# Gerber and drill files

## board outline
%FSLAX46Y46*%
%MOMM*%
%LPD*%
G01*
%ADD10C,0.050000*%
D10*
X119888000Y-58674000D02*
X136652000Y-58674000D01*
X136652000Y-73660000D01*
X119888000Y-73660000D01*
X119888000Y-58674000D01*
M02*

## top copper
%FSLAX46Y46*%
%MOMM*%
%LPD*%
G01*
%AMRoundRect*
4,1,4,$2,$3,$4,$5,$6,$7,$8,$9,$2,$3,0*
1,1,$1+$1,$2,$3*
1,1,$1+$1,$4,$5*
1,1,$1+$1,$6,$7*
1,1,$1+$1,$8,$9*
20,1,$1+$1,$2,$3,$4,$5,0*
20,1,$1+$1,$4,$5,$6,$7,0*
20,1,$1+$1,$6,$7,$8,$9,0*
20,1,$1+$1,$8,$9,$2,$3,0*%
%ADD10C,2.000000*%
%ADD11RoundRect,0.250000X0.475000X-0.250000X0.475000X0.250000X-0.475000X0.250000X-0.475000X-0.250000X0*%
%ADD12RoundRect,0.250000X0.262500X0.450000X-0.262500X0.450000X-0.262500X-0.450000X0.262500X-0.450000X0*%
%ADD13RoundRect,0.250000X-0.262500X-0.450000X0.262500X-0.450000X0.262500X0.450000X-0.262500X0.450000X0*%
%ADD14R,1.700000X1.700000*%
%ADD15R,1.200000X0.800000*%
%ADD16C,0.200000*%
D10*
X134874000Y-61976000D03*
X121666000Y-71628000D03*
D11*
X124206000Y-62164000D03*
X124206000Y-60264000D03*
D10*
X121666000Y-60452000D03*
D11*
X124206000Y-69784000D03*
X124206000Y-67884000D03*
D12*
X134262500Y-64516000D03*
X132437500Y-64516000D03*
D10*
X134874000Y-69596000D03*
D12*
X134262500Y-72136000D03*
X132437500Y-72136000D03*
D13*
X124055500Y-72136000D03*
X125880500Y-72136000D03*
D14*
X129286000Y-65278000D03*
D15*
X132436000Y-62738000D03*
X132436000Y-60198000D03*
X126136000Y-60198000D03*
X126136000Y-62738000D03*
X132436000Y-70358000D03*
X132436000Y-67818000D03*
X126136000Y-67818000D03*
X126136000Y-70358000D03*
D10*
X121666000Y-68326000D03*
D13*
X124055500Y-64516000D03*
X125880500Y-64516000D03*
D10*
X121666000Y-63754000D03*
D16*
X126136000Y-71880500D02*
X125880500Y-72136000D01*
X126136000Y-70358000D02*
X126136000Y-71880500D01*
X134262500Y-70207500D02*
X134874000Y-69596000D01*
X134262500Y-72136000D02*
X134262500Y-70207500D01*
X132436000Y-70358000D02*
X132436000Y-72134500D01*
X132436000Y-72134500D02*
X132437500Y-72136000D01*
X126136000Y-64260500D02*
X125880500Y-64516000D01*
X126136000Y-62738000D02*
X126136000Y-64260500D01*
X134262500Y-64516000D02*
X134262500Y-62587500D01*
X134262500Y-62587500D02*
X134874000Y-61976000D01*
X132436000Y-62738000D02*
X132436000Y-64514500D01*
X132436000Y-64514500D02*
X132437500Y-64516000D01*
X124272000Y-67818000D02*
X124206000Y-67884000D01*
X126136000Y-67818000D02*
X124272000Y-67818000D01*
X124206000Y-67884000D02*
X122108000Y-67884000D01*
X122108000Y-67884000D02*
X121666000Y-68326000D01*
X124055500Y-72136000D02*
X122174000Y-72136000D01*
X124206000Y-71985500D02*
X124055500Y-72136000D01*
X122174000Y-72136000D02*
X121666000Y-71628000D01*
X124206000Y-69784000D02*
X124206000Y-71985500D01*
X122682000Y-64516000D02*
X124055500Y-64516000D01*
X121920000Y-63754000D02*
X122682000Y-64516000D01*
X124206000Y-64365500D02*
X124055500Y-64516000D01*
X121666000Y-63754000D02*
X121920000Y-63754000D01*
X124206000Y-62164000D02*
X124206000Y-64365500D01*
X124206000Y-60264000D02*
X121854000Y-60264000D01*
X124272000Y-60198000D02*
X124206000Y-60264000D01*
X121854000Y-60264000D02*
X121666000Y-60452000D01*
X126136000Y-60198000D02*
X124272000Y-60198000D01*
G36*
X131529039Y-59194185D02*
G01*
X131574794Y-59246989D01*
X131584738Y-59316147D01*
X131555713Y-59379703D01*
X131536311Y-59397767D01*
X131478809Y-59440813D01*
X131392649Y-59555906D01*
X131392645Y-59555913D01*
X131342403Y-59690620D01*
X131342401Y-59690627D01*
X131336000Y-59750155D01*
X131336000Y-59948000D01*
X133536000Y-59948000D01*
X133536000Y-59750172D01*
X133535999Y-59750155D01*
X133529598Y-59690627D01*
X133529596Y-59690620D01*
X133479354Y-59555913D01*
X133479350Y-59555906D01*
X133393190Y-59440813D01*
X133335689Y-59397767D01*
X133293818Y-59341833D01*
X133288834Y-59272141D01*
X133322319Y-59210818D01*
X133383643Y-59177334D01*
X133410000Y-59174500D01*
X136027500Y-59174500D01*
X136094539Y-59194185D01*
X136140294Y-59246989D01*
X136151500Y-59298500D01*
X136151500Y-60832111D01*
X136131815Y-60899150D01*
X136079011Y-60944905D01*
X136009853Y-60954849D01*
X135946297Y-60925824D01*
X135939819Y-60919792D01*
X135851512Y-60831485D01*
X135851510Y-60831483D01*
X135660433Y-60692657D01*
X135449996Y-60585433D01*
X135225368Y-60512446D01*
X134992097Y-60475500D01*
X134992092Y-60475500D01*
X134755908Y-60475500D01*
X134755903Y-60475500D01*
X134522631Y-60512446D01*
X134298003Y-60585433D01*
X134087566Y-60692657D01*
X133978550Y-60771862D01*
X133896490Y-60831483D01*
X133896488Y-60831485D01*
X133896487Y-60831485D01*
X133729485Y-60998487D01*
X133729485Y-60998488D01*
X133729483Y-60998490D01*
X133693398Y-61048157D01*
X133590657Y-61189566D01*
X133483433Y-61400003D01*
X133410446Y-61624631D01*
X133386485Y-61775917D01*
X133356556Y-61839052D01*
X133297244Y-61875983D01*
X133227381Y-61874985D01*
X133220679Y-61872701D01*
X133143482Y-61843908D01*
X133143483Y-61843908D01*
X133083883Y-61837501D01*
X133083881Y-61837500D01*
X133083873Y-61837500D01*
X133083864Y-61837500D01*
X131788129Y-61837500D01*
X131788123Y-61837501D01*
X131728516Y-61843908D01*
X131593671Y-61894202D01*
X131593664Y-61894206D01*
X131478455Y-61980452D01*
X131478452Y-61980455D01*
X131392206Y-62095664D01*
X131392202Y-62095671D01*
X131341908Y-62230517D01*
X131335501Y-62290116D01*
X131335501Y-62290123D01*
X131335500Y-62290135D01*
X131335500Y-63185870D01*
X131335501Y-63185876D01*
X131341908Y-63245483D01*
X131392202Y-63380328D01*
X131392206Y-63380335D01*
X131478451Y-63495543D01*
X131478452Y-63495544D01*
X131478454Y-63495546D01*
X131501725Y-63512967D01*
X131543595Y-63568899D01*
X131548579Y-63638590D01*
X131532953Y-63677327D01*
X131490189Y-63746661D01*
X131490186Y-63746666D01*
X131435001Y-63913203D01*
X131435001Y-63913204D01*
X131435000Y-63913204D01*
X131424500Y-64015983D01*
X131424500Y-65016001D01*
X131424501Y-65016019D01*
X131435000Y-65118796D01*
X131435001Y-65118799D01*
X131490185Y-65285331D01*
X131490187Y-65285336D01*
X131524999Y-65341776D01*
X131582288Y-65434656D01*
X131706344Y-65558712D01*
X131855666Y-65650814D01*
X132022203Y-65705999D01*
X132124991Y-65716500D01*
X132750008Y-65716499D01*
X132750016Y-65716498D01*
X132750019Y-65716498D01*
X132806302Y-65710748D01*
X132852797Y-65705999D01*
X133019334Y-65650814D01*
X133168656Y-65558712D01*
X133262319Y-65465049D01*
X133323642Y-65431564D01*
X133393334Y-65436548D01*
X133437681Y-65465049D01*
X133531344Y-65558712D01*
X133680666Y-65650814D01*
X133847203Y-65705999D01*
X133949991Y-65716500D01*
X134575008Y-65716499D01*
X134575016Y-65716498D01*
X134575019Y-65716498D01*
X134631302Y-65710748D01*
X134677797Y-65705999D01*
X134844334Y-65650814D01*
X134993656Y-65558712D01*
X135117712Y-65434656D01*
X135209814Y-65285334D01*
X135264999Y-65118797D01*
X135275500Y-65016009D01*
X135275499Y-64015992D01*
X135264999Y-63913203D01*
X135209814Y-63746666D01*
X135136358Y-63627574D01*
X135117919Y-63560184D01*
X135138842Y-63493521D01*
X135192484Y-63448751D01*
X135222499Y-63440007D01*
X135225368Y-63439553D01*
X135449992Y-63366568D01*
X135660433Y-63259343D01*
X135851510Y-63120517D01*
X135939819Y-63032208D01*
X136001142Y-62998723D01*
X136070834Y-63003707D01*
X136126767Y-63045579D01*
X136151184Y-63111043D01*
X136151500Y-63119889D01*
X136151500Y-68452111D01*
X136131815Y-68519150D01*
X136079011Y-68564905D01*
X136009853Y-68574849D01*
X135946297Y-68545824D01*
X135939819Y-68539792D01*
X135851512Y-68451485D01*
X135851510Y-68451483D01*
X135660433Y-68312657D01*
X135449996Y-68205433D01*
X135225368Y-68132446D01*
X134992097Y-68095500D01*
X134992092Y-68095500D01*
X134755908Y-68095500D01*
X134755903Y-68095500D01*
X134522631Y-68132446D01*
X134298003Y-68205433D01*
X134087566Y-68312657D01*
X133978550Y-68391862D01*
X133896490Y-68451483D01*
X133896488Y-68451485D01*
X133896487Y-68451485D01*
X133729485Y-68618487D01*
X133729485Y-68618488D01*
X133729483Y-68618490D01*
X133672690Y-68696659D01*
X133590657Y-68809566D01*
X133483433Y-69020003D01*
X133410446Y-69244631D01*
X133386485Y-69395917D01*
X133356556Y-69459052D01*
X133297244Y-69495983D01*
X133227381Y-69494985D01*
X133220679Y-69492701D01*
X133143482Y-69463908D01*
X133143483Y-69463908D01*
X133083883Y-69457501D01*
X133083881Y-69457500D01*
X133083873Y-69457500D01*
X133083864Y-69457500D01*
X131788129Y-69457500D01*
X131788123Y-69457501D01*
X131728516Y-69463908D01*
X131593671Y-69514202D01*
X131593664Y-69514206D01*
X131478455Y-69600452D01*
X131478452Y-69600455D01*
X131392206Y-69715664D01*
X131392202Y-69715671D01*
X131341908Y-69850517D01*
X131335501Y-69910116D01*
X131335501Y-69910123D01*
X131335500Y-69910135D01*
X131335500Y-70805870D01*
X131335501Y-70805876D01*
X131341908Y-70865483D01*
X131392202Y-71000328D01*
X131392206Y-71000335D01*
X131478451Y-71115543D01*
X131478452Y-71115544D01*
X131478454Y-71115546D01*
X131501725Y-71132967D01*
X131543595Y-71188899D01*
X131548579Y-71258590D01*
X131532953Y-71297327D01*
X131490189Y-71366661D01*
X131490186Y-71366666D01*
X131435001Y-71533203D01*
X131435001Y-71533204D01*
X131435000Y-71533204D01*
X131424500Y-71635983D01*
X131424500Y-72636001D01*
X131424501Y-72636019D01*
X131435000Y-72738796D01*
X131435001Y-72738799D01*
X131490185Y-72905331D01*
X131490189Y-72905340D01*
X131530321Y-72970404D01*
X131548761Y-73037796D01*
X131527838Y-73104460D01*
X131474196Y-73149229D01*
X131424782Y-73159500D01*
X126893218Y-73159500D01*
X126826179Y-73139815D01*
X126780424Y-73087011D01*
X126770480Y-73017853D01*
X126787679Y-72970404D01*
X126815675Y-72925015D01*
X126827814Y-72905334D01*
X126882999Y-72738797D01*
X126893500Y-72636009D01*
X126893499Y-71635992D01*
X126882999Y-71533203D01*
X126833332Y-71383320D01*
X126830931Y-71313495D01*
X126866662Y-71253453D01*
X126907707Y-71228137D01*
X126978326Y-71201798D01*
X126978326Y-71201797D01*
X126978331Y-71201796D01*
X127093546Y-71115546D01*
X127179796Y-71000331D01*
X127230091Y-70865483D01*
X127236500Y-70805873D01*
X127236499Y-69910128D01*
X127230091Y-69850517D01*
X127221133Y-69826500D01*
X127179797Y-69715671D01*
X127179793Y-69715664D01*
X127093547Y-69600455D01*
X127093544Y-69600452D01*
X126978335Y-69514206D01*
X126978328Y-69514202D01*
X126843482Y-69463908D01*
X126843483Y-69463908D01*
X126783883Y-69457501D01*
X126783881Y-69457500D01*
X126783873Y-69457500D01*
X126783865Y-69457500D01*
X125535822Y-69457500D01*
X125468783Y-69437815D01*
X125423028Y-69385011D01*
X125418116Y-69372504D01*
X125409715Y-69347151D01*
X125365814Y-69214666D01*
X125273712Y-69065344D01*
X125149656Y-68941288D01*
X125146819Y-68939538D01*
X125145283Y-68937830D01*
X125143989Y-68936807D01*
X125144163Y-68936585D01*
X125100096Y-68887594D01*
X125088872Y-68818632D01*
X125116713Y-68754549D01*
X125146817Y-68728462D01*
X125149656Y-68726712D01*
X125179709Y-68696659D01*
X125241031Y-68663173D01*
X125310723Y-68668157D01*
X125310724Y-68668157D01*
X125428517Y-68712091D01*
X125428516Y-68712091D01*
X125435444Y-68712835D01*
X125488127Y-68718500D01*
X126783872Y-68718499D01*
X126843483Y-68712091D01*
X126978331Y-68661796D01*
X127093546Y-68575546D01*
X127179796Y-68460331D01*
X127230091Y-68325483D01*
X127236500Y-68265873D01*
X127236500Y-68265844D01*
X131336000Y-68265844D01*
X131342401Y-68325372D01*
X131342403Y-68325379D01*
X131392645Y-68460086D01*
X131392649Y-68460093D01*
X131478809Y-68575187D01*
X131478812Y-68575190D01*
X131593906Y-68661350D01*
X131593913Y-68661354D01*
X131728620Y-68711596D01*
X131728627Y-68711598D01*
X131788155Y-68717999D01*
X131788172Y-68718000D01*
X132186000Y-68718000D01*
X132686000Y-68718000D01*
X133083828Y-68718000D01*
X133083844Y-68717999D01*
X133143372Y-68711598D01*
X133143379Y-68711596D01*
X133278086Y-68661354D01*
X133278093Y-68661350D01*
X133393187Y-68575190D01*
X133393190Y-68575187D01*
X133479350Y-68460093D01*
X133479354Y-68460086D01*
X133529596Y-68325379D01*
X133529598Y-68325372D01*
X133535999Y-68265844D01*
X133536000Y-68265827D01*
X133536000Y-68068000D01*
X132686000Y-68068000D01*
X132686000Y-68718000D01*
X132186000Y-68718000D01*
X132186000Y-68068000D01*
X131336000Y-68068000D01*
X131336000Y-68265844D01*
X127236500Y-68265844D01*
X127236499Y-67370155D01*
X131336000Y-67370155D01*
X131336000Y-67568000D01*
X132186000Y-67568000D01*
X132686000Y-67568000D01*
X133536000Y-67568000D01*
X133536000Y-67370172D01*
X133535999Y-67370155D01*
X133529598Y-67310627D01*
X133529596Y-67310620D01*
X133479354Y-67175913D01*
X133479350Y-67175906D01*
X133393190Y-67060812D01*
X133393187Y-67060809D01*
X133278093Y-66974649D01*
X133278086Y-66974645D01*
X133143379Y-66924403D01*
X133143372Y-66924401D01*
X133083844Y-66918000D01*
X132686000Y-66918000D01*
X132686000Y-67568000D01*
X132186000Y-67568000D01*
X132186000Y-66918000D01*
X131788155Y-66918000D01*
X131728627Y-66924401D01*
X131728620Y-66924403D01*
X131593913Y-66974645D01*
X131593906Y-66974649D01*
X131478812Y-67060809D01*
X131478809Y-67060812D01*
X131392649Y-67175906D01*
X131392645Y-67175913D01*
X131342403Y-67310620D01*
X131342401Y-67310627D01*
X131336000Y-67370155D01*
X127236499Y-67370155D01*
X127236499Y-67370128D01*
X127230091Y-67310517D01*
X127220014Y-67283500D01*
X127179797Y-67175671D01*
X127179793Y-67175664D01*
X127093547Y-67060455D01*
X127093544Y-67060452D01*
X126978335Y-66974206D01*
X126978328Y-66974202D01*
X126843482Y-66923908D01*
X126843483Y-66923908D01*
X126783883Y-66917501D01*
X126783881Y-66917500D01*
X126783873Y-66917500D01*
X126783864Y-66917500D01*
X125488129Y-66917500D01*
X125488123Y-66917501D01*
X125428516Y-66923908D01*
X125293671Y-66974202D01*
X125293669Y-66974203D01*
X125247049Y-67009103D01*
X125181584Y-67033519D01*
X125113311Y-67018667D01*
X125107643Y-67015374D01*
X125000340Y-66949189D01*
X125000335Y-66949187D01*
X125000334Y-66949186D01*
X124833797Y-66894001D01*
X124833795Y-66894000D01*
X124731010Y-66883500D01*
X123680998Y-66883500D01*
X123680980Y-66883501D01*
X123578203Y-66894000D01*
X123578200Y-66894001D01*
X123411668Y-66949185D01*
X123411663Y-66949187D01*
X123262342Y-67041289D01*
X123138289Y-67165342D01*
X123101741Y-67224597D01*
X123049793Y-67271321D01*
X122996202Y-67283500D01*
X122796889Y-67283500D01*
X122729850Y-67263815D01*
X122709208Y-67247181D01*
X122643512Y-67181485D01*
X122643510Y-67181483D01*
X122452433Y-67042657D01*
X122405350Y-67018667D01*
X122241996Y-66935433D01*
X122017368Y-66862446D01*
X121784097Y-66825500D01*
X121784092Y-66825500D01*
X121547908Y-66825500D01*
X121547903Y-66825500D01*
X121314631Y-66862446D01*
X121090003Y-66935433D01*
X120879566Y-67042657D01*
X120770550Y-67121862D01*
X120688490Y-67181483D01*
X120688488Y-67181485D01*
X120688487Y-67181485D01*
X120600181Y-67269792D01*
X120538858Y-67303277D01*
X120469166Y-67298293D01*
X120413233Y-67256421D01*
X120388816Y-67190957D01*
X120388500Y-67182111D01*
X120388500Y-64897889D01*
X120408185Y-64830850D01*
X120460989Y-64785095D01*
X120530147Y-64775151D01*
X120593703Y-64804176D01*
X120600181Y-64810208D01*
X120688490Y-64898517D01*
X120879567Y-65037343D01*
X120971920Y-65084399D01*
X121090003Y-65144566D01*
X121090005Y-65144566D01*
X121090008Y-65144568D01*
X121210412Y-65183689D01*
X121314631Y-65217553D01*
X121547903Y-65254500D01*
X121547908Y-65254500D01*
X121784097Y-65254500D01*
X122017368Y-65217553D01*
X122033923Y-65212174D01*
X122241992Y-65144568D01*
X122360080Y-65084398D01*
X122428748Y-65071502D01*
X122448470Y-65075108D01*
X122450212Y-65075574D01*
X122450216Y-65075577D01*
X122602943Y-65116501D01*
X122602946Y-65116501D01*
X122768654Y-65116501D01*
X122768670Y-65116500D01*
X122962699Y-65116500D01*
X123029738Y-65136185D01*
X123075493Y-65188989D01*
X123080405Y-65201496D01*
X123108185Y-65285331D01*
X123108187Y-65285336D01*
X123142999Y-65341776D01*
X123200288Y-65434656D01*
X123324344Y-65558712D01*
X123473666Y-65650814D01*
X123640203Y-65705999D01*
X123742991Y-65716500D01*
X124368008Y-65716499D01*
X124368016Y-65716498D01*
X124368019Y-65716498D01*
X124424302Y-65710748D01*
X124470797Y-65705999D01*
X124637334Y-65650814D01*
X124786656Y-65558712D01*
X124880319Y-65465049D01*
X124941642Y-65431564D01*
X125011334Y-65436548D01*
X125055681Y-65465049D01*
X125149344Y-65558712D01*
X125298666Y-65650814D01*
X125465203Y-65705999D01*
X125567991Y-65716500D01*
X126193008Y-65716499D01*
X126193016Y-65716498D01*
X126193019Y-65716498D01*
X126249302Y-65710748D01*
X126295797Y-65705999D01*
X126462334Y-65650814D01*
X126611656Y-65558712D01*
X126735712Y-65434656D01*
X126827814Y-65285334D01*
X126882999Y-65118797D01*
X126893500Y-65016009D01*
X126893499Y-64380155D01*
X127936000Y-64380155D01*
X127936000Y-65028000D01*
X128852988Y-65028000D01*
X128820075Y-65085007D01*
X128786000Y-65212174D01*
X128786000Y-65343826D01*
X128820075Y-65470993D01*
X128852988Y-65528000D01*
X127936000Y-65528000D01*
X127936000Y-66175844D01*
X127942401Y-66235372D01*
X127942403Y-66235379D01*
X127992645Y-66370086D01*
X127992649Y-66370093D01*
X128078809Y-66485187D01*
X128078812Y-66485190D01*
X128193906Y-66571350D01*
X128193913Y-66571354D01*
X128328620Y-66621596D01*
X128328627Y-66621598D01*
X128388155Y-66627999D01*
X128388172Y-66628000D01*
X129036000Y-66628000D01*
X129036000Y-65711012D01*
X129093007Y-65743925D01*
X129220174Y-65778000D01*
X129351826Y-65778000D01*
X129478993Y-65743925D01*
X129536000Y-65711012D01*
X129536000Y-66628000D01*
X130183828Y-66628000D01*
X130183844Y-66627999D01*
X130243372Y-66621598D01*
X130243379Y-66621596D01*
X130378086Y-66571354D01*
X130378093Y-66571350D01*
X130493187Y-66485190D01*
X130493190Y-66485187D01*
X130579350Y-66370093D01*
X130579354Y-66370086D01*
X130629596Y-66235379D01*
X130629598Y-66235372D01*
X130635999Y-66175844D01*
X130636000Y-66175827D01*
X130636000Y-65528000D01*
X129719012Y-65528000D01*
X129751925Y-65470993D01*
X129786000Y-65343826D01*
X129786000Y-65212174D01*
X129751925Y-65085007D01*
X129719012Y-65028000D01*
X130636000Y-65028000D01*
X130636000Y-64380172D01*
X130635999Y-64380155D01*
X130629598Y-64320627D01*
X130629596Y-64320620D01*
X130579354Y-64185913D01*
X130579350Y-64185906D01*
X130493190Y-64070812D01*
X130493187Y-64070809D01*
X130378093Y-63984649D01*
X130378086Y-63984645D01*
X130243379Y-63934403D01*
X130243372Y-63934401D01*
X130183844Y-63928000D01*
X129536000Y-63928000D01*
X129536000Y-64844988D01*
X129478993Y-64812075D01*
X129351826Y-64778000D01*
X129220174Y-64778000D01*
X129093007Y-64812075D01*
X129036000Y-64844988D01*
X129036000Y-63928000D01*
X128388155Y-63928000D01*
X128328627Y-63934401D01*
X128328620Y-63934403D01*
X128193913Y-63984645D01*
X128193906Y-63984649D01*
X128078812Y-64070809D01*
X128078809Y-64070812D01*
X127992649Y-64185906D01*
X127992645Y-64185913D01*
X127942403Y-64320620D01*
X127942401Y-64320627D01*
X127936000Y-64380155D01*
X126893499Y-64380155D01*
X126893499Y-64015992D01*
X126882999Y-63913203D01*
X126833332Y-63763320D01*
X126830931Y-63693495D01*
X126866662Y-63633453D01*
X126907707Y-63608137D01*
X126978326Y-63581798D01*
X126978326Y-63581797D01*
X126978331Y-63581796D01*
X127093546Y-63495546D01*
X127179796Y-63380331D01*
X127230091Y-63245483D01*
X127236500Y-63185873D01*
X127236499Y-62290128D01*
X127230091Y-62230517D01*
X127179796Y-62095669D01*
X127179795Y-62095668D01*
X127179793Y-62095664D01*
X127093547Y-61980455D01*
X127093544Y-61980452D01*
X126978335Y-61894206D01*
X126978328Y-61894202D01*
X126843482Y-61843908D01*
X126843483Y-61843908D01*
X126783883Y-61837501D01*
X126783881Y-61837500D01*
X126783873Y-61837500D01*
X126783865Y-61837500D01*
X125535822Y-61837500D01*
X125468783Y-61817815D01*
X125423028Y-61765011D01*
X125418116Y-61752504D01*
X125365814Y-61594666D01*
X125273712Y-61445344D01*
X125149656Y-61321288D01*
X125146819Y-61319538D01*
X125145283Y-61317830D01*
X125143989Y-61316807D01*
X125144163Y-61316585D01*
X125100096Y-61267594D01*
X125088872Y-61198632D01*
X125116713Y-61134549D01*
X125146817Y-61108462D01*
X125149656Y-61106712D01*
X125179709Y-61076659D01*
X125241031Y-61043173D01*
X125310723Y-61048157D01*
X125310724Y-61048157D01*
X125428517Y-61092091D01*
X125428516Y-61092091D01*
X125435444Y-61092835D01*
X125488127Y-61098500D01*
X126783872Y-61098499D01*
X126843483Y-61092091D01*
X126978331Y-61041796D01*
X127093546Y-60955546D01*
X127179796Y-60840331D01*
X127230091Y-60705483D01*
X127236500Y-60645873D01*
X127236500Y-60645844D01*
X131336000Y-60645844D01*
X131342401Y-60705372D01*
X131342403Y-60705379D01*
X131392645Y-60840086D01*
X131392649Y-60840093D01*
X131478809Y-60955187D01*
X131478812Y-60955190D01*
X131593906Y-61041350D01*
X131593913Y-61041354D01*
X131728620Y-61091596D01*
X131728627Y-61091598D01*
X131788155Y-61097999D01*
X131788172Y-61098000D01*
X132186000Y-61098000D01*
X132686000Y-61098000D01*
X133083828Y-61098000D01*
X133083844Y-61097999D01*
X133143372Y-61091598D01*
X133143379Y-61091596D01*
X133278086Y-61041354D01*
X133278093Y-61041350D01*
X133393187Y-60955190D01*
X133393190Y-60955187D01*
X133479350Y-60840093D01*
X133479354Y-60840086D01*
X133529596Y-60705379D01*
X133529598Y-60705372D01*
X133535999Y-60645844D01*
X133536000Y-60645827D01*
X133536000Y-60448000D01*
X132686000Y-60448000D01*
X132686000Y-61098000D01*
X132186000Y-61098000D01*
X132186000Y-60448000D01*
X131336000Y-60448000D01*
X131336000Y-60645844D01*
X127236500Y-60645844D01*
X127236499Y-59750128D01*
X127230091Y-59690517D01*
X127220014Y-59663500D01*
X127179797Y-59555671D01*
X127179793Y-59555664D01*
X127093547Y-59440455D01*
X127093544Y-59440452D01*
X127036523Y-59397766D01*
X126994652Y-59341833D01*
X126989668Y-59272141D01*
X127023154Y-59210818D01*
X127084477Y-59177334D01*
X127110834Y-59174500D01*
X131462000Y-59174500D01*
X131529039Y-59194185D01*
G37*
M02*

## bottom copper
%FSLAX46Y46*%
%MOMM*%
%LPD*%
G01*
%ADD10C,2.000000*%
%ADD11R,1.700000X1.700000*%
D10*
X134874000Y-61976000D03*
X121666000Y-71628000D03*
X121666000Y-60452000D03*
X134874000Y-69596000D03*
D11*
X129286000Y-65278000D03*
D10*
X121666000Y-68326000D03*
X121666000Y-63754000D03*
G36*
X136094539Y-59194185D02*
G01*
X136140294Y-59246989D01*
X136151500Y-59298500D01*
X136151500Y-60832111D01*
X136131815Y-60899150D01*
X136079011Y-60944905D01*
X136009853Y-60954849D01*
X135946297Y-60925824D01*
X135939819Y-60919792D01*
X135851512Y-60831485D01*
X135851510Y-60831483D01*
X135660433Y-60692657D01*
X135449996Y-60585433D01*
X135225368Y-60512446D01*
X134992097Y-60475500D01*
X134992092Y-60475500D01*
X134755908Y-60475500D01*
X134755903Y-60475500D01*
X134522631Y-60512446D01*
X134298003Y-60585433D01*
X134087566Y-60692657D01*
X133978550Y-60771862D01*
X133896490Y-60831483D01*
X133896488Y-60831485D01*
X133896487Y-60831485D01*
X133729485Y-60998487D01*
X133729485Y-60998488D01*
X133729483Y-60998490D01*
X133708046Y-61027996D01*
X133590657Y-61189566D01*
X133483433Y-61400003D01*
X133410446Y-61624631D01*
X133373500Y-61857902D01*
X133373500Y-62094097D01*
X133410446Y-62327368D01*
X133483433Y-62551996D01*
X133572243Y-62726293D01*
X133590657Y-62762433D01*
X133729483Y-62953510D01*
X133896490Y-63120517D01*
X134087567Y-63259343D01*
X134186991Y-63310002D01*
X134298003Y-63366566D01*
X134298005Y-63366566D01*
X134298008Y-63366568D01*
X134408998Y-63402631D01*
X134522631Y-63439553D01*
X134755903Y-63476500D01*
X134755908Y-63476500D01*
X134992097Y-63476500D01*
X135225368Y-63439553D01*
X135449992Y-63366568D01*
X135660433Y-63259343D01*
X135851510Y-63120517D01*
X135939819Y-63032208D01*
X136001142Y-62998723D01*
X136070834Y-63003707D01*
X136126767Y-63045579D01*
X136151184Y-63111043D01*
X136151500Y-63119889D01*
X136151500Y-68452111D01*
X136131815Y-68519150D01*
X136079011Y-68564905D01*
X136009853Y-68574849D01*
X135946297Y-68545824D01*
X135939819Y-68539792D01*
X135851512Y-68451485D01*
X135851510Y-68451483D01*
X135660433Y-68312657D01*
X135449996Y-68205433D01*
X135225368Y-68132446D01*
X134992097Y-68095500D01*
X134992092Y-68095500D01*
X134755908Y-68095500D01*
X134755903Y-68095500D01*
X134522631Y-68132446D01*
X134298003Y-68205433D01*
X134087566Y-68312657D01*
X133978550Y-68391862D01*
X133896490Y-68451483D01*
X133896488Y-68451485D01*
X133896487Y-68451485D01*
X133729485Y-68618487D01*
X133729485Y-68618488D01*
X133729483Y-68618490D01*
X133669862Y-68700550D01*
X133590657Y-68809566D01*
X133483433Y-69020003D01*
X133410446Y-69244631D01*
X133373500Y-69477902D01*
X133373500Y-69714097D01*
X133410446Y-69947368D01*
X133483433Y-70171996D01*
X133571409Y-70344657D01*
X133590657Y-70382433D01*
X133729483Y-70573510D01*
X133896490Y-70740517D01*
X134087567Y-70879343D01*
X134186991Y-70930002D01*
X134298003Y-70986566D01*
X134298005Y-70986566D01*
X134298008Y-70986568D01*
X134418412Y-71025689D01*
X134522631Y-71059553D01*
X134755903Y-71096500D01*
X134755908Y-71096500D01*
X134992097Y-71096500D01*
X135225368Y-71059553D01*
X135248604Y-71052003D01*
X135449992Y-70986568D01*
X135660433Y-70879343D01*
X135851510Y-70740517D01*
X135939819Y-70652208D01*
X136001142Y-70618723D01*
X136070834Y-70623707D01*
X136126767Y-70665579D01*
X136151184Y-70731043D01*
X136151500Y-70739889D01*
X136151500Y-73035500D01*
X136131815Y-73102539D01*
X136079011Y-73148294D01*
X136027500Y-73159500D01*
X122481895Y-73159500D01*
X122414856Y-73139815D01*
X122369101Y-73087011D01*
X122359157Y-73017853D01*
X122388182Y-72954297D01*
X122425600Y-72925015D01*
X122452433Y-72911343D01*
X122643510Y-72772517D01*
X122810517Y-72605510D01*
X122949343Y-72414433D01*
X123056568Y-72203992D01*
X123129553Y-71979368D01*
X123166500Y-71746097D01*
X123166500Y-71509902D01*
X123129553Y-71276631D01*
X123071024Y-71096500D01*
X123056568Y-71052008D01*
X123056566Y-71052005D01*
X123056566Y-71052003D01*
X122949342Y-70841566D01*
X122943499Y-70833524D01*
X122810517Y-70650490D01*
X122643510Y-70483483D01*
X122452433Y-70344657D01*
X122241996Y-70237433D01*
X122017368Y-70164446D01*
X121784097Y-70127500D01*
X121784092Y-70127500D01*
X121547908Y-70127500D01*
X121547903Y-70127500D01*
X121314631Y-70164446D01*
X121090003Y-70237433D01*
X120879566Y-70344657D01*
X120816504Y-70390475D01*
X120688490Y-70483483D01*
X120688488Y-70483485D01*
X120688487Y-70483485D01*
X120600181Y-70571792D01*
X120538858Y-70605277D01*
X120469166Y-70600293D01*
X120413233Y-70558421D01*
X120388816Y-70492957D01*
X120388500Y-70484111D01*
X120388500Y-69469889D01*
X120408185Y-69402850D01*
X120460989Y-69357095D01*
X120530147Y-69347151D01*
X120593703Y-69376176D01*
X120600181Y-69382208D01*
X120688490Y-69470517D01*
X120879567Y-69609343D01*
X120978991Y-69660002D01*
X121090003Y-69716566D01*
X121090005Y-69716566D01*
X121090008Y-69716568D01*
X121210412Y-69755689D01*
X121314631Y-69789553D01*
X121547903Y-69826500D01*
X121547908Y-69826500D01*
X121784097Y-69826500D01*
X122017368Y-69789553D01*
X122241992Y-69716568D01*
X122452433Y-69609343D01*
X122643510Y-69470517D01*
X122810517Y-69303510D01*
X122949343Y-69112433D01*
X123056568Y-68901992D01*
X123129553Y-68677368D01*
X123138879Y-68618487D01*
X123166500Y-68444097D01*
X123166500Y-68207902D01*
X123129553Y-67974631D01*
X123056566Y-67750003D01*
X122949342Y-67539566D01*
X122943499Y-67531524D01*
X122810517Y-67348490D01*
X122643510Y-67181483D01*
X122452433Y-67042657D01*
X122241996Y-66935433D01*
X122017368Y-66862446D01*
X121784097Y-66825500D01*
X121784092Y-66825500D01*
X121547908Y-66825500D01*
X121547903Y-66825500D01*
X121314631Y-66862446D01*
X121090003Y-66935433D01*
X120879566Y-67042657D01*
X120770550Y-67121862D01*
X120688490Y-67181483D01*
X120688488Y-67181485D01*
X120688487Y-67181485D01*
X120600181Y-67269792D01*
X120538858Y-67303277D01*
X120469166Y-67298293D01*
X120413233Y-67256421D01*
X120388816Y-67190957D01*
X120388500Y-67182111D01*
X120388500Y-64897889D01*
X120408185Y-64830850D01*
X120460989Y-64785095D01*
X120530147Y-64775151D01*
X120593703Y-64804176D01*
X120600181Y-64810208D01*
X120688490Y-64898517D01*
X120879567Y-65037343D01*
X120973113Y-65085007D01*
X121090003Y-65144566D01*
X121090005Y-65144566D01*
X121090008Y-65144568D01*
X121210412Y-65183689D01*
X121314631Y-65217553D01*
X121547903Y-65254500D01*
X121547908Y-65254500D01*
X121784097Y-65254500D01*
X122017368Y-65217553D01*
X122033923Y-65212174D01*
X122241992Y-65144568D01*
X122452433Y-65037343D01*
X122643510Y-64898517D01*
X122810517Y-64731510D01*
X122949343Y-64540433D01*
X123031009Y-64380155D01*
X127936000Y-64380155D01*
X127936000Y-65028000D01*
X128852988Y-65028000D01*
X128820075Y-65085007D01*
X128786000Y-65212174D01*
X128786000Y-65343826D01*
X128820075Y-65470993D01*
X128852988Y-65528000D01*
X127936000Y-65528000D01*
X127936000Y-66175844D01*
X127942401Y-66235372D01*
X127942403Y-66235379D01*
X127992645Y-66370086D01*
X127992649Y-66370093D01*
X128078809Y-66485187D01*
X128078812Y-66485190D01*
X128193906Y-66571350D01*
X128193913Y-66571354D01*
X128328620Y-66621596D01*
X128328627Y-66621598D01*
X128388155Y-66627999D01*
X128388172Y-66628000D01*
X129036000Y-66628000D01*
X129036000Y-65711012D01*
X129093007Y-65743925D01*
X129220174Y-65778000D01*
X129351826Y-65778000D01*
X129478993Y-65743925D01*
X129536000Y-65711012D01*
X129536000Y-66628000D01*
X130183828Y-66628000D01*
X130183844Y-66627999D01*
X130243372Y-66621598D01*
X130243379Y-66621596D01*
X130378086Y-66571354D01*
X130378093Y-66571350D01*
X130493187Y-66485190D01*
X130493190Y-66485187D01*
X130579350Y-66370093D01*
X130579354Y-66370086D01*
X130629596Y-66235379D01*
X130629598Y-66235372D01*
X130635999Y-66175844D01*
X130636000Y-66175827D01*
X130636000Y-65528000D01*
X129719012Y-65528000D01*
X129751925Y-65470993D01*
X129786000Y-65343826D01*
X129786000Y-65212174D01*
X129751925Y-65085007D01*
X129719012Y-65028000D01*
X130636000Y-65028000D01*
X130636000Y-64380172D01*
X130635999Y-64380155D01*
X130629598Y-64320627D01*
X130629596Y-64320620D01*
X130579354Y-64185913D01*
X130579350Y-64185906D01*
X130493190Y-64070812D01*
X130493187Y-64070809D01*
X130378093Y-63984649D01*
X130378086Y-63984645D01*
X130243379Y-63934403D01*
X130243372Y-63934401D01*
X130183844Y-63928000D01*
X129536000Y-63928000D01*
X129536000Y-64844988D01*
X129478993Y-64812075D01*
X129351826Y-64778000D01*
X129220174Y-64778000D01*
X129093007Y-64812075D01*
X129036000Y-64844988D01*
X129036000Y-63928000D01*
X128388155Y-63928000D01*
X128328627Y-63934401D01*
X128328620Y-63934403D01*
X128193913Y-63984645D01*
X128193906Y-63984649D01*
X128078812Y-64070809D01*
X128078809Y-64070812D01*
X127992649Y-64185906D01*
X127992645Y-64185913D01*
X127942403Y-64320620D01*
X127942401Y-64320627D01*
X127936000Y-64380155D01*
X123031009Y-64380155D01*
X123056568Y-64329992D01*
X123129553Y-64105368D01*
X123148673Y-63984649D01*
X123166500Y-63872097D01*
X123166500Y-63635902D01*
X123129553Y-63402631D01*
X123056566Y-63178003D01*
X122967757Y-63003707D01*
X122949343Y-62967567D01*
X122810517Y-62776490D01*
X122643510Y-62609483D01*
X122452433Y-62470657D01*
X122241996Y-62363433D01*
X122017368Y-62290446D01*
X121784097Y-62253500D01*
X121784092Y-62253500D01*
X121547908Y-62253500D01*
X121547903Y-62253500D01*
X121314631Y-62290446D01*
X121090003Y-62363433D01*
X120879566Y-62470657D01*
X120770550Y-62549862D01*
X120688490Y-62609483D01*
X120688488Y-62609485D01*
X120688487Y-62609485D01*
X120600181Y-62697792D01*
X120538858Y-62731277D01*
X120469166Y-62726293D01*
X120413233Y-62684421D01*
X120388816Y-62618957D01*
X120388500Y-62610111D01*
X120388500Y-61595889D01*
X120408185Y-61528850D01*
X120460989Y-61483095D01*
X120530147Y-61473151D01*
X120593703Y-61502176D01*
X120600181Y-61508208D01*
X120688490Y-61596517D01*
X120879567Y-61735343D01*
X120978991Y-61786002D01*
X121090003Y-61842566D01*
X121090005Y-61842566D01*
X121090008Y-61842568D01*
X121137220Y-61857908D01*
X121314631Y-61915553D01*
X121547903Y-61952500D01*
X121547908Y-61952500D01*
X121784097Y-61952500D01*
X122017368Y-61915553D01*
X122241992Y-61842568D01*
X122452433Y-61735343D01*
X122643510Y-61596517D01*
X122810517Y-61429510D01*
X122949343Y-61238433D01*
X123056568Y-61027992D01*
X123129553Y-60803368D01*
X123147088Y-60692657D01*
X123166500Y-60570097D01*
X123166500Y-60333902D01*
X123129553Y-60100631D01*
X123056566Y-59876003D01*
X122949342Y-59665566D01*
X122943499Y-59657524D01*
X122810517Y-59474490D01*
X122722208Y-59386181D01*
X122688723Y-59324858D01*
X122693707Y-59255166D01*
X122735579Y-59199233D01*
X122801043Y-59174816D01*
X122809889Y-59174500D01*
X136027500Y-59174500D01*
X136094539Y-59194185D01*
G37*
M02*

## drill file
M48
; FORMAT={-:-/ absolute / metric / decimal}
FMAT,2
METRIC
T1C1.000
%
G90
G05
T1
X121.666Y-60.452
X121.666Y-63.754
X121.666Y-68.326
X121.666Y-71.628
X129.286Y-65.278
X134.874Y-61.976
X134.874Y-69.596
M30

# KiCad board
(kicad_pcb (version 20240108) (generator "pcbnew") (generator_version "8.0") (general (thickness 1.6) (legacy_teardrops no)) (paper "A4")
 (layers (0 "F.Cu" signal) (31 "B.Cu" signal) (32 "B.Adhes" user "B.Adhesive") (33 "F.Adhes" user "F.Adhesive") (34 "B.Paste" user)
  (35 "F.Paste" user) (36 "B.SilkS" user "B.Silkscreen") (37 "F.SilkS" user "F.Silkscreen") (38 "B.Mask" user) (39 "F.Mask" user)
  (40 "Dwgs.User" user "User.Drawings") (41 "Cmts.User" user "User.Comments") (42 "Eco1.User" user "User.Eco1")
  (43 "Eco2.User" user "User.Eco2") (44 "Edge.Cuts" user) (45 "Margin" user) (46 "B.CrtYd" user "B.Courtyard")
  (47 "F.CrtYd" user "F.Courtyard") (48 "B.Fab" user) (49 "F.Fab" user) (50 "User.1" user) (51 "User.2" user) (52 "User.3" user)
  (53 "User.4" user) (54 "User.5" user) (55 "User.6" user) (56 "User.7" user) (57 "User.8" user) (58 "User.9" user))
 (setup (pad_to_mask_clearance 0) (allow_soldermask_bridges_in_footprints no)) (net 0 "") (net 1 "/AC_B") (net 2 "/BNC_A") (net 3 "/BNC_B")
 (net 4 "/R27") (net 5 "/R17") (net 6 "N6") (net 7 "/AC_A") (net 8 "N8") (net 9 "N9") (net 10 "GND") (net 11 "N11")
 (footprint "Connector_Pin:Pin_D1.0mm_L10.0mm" (layer "F.Cu") (at 134.874 61.976 180)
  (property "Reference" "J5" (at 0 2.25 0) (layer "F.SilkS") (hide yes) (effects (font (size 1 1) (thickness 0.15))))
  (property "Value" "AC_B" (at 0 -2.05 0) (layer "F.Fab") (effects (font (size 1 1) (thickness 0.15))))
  (pad "1" thru_hole circle (at 0 0 180) (size 2 2) (drill 1) (layers "*.Cu" "*.Mask") (remove_unused_layers no) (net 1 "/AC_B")))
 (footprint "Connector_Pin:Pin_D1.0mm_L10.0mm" (layer "F.Cu") (at 121.666 71.628 180)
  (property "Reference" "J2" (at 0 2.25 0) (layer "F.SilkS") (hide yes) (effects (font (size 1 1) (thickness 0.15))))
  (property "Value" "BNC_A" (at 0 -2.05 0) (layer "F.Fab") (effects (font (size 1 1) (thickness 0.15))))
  (pad "1" thru_hole circle (at 0 0 180) (size 2 2) (drill 1) (layers "*.Cu" "*.Mask") (remove_unused_layers no) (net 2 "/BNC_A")))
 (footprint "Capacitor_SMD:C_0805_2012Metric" (layer "F.Cu") (at 124.206 61.214 90)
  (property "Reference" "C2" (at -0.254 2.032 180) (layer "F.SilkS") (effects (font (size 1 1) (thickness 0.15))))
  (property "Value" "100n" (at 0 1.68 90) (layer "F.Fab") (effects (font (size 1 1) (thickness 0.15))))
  (pad "1" smd roundrect (at -0.95 0 90) (size 1 1.45) (layers "F.Cu" "F.Paste" "F.Mask") (roundrect_rratio 0.25) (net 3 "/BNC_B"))
  (pad "2" smd roundrect (at 0.95 0 90) (size 1 1.45) (layers "F.Cu" "F.Paste" "F.Mask") (roundrect_rratio 0.25) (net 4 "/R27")))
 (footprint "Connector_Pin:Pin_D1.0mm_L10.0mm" (layer "F.Cu") (at 121.666 60.452 180)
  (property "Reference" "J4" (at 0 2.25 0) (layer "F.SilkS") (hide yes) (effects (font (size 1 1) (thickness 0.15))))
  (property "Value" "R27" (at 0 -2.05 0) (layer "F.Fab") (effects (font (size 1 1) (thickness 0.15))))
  (pad "1" thru_hole circle (at 0 0 180) (size 2 2) (drill 1) (layers "*.Cu" "*.Mask") (remove_unused_layers no) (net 4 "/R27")))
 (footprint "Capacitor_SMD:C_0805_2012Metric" (layer "F.Cu") (at 124.206 68.834 90)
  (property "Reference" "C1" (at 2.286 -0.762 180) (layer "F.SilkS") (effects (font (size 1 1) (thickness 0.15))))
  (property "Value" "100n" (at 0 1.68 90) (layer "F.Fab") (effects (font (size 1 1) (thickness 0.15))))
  (pad "1" smd roundrect (at -0.95 0 90) (size 1 1.45) (layers "F.Cu" "F.Paste" "F.Mask") (roundrect_rratio 0.25) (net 2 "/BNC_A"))
  (pad "2" smd roundrect (at 0.95 0 90) (size 1 1.45) (layers "F.Cu" "F.Paste" "F.Mask") (roundrect_rratio 0.25) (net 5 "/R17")))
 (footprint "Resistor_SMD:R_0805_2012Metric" (layer "F.Cu") (at 133.35 64.516 180)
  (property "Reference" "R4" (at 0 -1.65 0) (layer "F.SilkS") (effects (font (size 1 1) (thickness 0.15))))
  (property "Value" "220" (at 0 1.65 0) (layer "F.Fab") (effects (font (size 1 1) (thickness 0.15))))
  (pad "1" smd roundrect (at -0.9125 0 180) (size 1.025 1.4) (layers "F.Cu" "F.Paste" "F.Mask") (roundrect_rratio 0.243902) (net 1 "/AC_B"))
  (pad "2" smd roundrect (at 0.9125 0 180) (size 1.025 1.4) (layers "F.Cu" "F.Paste" "F.Mask") (roundrect_rratio 0.243902) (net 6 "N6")))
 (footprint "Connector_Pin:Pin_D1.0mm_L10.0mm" (layer "F.Cu") (at 134.874 69.596 180)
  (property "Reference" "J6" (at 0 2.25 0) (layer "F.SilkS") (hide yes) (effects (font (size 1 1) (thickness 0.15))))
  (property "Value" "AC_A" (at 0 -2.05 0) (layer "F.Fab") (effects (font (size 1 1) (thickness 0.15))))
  (pad "1" thru_hole circle (at 0 0 180) (size 2 2) (drill 1) (layers "*.Cu" "*.Mask") (remove_unused_layers no) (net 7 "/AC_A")))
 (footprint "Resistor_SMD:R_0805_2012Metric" (layer "F.Cu") (at 133.35 72.136 180)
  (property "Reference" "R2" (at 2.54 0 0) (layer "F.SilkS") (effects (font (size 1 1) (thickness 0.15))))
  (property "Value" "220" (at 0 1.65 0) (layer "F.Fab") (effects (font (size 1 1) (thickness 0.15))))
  (pad "1" smd roundrect (at -0.9125 0 180) (size 1.025 1.4) (layers "F.Cu" "F.Paste" "F.Mask") (roundrect_rratio 0.243902) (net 7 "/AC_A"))
  (pad "2" smd roundrect (at 0.9125 0 180) (size 1.025 1.4) (layers "F.Cu" "F.Paste" "F.Mask") (roundrect_rratio 0.243902) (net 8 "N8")))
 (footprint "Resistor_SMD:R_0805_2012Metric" (layer "F.Cu") (at 124.968 72.136)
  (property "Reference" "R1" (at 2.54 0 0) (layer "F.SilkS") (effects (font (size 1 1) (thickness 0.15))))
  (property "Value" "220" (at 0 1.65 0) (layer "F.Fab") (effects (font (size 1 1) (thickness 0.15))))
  (pad "1" smd roundrect (at -0.9125 0) (size 1.025 1.4) (layers "F.Cu" "F.Paste" "F.Mask") (roundrect_rratio 0.243902) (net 2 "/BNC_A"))
  (pad "2" smd roundrect (at 0.9125 0) (size 1.025 1.4) (layers "F.Cu" "F.Paste" "F.Mask") (roundrect_rratio 0.243902) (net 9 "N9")))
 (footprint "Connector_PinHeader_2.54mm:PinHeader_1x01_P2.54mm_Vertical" (layer "F.Cu") (at 129.286 65.278)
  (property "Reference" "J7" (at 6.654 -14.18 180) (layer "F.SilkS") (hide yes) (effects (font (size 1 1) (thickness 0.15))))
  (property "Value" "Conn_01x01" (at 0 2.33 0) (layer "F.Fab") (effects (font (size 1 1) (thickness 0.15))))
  (pad "1" thru_hole rect (at 0 0) (size 1.7 1.7) (drill 1) (layers "*.Cu" "*.Mask") (remove_unused_layers no) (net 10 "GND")))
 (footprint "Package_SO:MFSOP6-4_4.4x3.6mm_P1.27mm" (layer "F.Cu") (at 129.286 61.468 180)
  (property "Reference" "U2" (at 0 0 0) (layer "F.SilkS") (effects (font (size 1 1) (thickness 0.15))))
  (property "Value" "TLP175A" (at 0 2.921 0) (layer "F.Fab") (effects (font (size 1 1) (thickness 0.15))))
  (pad "1" smd rect (at -3.15 -1.27 180) (size 1.2 0.8) (layers "F.Cu" "F.Paste" "F.Mask") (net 6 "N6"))
  (pad "3" smd rect (at -3.15 1.27 180) (size 1.2 0.8) (layers "F.Cu" "F.Paste" "F.Mask") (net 10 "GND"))
  (pad "4" smd rect (at 3.15 1.27 180) (size 1.2 0.8) (layers "F.Cu" "F.Paste" "F.Mask") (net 4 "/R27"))
  (pad "6" smd rect (at 3.15 -1.27 180) (size 1.2 0.8) (layers "F.Cu" "F.Paste" "F.Mask") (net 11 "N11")))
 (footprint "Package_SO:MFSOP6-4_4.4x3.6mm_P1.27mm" (layer "F.Cu") (at 129.286 69.088 180)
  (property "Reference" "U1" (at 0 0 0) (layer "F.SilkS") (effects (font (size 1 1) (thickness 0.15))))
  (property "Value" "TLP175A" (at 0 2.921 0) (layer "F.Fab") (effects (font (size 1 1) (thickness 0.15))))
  (pad "1" smd rect (at -3.15 -1.27 180) (size 1.2 0.8) (layers "F.Cu" "F.Paste" "F.Mask") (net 8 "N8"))
  (pad "3" smd rect (at -3.15 1.27 180) (size 1.2 0.8) (layers "F.Cu" "F.Paste" "F.Mask") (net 10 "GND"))
  (pad "4" smd rect (at 3.15 1.27 180) (size 1.2 0.8) (layers "F.Cu" "F.Paste" "F.Mask") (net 5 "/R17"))
  (pad "6" smd rect (at 3.15 -1.27 180) (size 1.2 0.8) (layers "F.Cu" "F.Paste" "F.Mask") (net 9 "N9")))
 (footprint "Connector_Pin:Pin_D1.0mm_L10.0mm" (layer "F.Cu") (at 121.666 68.326 180)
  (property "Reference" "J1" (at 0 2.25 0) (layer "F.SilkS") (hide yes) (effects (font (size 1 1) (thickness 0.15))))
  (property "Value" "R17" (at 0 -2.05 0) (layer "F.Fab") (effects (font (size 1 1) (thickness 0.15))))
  (pad "1" thru_hole circle (at 0 0 180) (size 2 2) (drill 1) (layers "*.Cu" "*.Mask") (remove_unused_layers no) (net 5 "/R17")))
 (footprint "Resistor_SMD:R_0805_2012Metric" (layer "F.Cu") (at 124.968 64.516)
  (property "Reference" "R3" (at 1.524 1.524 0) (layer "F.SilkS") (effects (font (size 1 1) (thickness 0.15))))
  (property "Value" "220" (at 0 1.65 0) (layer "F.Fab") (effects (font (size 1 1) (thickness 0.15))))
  (pad "1" smd roundrect (at -0.9125 0) (size 1.025 1.4) (layers "F.Cu" "F.Paste" "F.Mask") (roundrect_rratio 0.243902) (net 3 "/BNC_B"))
  (pad "2" smd roundrect (at 0.9125 0) (size 1.025 1.4) (layers "F.Cu" "F.Paste" "F.Mask") (roundrect_rratio 0.243902) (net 11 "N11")))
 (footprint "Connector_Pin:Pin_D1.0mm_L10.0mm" (layer "F.Cu") (at 121.666 63.754 180)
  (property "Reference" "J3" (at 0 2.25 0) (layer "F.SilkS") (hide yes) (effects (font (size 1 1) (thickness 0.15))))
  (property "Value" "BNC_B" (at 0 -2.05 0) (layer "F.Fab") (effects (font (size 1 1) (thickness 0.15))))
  (pad "1" thru_hole circle (at 0 0 180) (size 2 2) (drill 1) (layers "*.Cu" "*.Mask") (remove_unused_layers no) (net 3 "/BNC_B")))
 (gr_rect (start 119.888 58.674) (end 136.652 73.66) (stroke (width 0.05) (type default)) (fill none) (layer "Edge.Cuts"))
 (segment (start 126.136 71.8805) (end 125.8805 72.136) (width 0.2) (layer "F.Cu") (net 9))
 (segment (start 126.136 70.358) (end 126.136 71.8805) (width 0.2) (layer "F.Cu") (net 9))
 (segment (start 134.2625 70.2075) (end 134.874 69.596) (width 0.2) (layer "F.Cu") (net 7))
 (segment (start 134.2625 72.136) (end 134.2625 70.2075) (width 0.2) (layer "F.Cu") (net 7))
 (segment (start 132.436 70.358) (end 132.436 72.1345) (width 0.2) (layer "F.Cu") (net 8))
 (segment (start 132.436 72.1345) (end 132.4375 72.136) (width 0.2) (layer "F.Cu") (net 8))
 (segment (start 126.136 64.2605) (end 125.8805 64.516) (width 0.2) (layer "F.Cu") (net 11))
 (segment (start 126.136 62.738) (end 126.136 64.2605) (width 0.2) (layer "F.Cu") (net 11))
 (segment (start 134.2625 64.516) (end 134.2625 62.5875) (width 0.2) (layer "F.Cu") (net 1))
 (segment (start 134.2625 62.5875) (end 134.874 61.976) (width 0.2) (layer "F.Cu") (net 1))
 (segment (start 132.436 62.738) (end 132.436 64.5145) (width 0.2) (layer "F.Cu") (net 6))
 (segment (start 132.436 64.5145) (end 132.4375 64.516) (width 0.2) (layer "F.Cu") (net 6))
 (segment (start 124.272 67.818) (end 124.206 67.884) (width 0.2) (layer "F.Cu") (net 5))
 (segment (start 126.136 67.818) (end 124.272 67.818) (width 0.2) (layer "F.Cu") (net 5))
 (segment (start 124.206 67.884) (end 122.108 67.884) (width 0.2) (layer "F.Cu") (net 5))
 (segment (start 122.108 67.884) (end 121.666 68.326) (width 0.2) (layer "F.Cu") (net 5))
 (segment (start 124.0555 72.136) (end 122.174 72.136) (width 0.2) (layer "F.Cu") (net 2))
 (segment (start 124.206 71.9855) (end 124.0555 72.136) (width 0.2) (layer "F.Cu") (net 2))
 (segment (start 122.174 72.136) (end 121.666 71.628) (width 0.2) (layer "F.Cu") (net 2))
 (segment (start 124.206 69.784) (end 124.206 71.9855) (width 0.2) (layer "F.Cu") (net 2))
 (segment (start 122.682 64.516) (end 124.0555 64.516) (width 0.2) (layer "F.Cu") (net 3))
 (segment (start 121.92 63.754) (end 122.682 64.516) (width 0.2) (layer "F.Cu") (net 3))
 (segment (start 124.206 64.3655) (end 124.0555 64.516) (width 0.2) (layer "F.Cu") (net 3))
 (segment (start 121.666 63.754) (end 121.92 63.754) (width 0.2) (layer "F.Cu") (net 3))
 (segment (start 124.206 62.164) (end 124.206 64.3655) (width 0.2) (layer "F.Cu") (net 3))
 (segment (start 124.206 60.264) (end 121.854 60.264) (width 0.2) (layer "F.Cu") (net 4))
 (segment (start 124.272 60.198) (end 124.206 60.264) (width 0.2) (layer "F.Cu") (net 4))
 (segment (start 121.854 60.264) (end 121.666 60.452) (width 0.2) (layer "F.Cu") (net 4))
 (segment (start 126.136 60.198) (end 124.272 60.198) (width 0.2) (layer "F.Cu") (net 4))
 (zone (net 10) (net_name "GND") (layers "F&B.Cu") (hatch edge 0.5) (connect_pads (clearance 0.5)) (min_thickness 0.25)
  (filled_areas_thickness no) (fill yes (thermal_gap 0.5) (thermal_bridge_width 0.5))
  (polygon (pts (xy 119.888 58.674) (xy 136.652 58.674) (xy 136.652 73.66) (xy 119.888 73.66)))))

